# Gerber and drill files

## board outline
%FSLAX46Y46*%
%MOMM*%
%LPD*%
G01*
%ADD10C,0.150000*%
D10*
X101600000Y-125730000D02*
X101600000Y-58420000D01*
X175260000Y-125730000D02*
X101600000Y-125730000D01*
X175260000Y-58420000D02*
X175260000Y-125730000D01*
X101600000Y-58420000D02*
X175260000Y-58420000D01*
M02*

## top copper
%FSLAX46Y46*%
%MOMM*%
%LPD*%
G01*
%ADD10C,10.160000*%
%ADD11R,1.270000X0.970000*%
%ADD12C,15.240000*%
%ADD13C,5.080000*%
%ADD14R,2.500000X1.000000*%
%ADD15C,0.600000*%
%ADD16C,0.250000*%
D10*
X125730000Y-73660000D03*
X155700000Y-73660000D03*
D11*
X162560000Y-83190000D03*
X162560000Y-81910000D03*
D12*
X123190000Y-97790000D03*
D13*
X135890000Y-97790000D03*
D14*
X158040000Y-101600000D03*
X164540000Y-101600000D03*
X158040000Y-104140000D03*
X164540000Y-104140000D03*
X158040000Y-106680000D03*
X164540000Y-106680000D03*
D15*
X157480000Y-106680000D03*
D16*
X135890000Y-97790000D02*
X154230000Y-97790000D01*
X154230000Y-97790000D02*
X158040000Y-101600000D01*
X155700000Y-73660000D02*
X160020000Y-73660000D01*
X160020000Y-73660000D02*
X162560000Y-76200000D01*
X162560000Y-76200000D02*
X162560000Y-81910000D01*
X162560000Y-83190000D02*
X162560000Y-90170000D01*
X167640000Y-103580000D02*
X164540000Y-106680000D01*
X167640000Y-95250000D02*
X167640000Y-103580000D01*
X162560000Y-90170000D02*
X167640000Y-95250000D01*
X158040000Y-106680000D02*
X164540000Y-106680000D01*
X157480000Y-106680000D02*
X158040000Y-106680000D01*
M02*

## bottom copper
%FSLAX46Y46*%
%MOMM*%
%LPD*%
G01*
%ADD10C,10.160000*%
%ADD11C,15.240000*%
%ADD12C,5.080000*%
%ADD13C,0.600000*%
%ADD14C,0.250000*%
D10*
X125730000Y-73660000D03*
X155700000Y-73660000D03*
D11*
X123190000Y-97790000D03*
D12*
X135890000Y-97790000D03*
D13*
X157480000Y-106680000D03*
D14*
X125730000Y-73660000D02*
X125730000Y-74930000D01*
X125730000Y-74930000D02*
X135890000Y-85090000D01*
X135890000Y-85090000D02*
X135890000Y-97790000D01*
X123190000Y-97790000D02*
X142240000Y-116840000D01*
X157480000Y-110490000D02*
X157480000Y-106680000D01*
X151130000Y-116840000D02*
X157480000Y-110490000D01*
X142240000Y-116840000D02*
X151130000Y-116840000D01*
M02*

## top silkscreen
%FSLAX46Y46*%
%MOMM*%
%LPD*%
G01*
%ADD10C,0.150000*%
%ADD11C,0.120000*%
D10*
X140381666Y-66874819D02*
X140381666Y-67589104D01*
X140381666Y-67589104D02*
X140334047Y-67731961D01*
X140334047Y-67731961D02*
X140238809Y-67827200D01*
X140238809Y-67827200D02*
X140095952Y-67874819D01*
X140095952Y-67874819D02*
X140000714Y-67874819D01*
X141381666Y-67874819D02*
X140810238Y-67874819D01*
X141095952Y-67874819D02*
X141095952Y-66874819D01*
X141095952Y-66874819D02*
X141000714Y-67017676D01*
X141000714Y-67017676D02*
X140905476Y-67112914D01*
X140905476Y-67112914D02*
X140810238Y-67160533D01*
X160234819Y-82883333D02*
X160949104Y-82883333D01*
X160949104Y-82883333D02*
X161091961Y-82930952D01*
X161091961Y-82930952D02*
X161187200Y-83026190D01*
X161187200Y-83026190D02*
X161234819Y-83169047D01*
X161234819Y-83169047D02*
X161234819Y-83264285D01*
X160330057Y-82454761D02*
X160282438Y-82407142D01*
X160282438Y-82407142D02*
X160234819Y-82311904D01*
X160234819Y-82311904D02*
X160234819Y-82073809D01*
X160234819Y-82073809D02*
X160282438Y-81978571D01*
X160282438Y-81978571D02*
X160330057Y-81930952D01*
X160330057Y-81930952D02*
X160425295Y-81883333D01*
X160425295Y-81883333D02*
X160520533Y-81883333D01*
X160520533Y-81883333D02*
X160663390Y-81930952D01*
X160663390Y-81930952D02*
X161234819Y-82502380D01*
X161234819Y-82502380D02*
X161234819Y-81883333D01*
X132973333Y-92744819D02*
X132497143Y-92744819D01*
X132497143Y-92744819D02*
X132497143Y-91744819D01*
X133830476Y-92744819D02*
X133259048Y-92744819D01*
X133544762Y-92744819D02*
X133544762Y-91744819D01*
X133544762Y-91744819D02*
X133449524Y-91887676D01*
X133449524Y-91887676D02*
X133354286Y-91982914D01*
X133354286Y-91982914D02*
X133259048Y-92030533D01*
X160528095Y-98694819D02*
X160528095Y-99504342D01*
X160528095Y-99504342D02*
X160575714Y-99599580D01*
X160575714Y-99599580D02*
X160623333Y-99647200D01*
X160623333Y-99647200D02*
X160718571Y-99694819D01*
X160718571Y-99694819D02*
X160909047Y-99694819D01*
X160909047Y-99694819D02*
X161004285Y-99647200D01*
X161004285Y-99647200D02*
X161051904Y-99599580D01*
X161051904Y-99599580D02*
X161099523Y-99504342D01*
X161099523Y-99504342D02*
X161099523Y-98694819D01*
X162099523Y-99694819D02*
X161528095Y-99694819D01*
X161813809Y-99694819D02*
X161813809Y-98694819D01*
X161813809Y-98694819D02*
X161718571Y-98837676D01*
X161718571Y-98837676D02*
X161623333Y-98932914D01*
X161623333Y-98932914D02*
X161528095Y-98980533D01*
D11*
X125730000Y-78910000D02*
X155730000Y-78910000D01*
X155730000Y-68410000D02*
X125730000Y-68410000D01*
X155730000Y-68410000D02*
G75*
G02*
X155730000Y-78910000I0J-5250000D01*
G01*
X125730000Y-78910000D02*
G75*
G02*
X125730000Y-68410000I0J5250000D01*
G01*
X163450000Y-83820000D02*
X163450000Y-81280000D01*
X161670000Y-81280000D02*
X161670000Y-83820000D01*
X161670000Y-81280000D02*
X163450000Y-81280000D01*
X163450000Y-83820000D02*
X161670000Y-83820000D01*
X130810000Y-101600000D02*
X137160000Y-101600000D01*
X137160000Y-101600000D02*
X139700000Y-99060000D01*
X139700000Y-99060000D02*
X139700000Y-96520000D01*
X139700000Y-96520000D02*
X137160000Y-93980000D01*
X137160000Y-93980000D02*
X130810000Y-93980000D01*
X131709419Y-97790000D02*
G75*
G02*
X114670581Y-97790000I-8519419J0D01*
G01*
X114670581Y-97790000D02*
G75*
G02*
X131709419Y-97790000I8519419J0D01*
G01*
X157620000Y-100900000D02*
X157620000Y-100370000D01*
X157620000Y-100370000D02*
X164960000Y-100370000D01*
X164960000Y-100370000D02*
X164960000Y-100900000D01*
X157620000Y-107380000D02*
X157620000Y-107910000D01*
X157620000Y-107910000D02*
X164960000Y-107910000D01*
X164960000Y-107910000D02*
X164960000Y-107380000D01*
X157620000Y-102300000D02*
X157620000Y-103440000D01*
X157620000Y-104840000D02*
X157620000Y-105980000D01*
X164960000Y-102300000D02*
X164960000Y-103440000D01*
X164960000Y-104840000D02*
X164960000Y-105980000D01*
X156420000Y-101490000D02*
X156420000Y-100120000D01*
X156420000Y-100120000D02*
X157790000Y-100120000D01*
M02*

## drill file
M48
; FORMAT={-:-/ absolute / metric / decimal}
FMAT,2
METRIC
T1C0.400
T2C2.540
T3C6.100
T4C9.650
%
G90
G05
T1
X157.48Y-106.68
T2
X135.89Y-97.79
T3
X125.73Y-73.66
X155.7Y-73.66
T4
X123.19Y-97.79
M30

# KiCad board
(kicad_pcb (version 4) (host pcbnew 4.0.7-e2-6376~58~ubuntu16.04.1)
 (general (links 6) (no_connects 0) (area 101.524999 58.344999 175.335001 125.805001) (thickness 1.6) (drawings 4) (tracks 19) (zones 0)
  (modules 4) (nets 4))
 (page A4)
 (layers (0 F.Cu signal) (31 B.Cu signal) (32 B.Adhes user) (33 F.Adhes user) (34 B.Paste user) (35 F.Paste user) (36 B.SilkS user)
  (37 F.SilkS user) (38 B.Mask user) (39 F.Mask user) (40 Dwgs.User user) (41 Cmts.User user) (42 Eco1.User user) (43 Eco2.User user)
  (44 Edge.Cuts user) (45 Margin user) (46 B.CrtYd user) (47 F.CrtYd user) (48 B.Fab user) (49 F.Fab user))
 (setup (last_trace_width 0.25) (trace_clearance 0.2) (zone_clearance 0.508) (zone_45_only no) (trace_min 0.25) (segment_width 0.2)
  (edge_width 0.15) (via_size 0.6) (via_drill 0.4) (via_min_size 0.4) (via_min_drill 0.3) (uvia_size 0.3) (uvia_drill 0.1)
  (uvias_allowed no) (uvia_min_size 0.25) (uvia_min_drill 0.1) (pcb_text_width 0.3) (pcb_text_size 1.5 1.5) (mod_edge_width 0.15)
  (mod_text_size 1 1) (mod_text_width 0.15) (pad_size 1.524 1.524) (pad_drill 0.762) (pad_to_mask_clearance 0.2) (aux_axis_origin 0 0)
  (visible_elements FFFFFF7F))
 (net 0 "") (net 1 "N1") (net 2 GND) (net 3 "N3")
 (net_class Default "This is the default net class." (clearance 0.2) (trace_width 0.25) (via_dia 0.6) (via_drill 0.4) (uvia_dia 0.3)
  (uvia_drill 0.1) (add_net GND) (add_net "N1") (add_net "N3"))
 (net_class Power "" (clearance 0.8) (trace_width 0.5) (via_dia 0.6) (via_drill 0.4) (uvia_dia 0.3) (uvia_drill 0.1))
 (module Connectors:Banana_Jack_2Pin (layer F.Cu) (at 125.73 73.66)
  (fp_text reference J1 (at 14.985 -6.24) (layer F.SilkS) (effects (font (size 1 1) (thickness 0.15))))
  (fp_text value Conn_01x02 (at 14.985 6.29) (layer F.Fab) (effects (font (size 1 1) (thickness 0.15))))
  (fp_line (start 0 5.25) (end 30 5.25) (layer F.SilkS) (width 0.12))
  (fp_line (start 30 -5.25) (end 0 -5.25) (layer F.SilkS) (width 0.12))
  (fp_arc (start 30 0) (end 30 -5.25) (angle 180) (layer F.SilkS) (width 0.12))
  (fp_arc (start 0 0) (end 0 5.25) (angle 180) (layer F.SilkS) (width 0.12))
  (pad 1 thru_hole circle (at 0 0) (size 10.16 10.16) (drill 6.1) (layers *.Cu *.Mask) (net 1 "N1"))
  (pad 2 thru_hole circle (at 29.97 0) (size 10.16 10.16) (drill 6.1) (layers *.Cu *.Mask) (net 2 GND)))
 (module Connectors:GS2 (layer F.Cu) (at 162.56 82.55 180)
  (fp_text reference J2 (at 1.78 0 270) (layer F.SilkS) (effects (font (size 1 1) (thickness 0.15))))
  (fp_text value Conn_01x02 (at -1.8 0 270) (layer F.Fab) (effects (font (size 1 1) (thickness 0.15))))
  (fp_line (start -0.89 -1.27) (end -0.89 1.27) (layer F.SilkS) (width 0.12))
  (fp_line (start 0.89 1.27) (end 0.89 -1.27) (layer F.SilkS) (width 0.12))
  (fp_line (start 0.89 1.27) (end -0.89 1.27) (layer F.SilkS) (width 0.12))
  (fp_line (start -0.89 -1.27) (end 0.89 -1.27) (layer F.SilkS) (width 0.12))
  (pad 1 smd rect (at 0 -0.64 180) (size 1.27 0.97) (layers F.Cu F.Paste F.Mask) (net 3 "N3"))
  (pad 2 smd rect (at 0 0.64 180) (size 1.27 0.97) (layers F.Cu F.Paste F.Mask) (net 2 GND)))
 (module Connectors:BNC (layer F.Cu) (at 135.89 97.79)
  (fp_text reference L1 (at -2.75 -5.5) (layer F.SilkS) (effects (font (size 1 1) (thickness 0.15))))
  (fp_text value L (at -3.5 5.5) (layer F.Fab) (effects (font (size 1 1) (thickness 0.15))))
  (fp_line (start -5.08 3.81) (end 1.27 3.81) (layer F.SilkS) (width 0.12))
  (fp_line (start 1.27 3.81) (end 3.81 1.27) (layer F.SilkS) (width 0.12))
  (fp_line (start 3.81 1.27) (end 3.81 -1.27) (layer F.SilkS) (width 0.12))
  (fp_line (start 3.81 -1.27) (end 1.27 -3.81) (layer F.SilkS) (width 0.12))
  (fp_line (start 1.27 -3.81) (end -5.08 -3.81) (layer F.SilkS) (width 0.12))
  (fp_circle (center -12.7 0) (end -5.08 3.81) (layer F.SilkS) (width 0.12))
  (pad 2 thru_hole circle (at -12.7 0) (size 15.24 15.24) (drill 9.65) (layers *.Cu *.Mask) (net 3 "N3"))
  (pad 1 thru_hole circle (at 0 0) (size 5.08 5.08) (drill 2.54) (layers *.Cu *.Mask) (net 1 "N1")))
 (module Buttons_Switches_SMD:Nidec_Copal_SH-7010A (layer F.Cu) (at 161.29 104.14)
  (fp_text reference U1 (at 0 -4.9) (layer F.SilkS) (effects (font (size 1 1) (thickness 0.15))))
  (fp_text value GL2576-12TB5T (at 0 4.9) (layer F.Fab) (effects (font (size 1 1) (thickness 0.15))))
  (fp_line (start -3.67 -3.24) (end -3.67 -3.77) (layer F.SilkS) (width 0.12))
  (fp_line (start -3.67 -3.77) (end 3.67 -3.77) (layer F.SilkS) (width 0.12))
  (fp_line (start 3.67 -3.77) (end 3.67 -3.24) (layer F.SilkS) (width 0.12))
  (fp_line (start -3.67 3.24) (end -3.67 3.77) (layer F.SilkS) (width 0.12))
  (fp_line (start -3.67 3.77) (end 3.67 3.77) (layer F.SilkS) (width 0.12))
  (fp_line (start 3.67 3.77) (end 3.67 3.24) (layer F.SilkS) (width 0.12))
  (fp_line (start -3.67 -1.84) (end -3.67 -0.7) (layer F.SilkS) (width 0.12))
  (fp_line (start -3.67 0.7) (end -3.67 1.84) (layer F.SilkS) (width 0.12))
  (fp_line (start 3.67 -1.84) (end 3.67 -0.7) (layer F.SilkS) (width 0.12))
  (fp_line (start 3.67 0.7) (end 3.67 1.84) (layer F.SilkS) (width 0.12))
  (fp_line (start -4.87 -2.65) (end -4.87 -4.02) (layer F.SilkS) (width 0.12))
  (fp_line (start -4.87 -4.02) (end -3.5 -4.02) (layer F.SilkS) (width 0.12))
  (pad 1 smd rect (at -3.25 -2.54) (size 2.5 1) (layers F.Cu F.Paste F.Mask) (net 1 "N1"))
  (pad 8 smd rect (at 3.25 -2.54) (size 2.5 1) (layers F.Cu F.Paste F.Mask))
  (pad C smd rect (at -3.25 0) (size 2.5 1) (layers F.Cu F.Paste F.Mask))
  (pad C smd rect (at 3.25 0) (size 2.5 1) (layers F.Cu F.Paste F.Mask))
  (pad 4 smd rect (at -3.25 2.54) (size 2.5 1) (layers F.Cu F.Paste F.Mask) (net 3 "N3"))
  (pad 2 smd rect (at 3.25 2.54) (size 2.5 1) (layers F.Cu F.Paste F.Mask) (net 3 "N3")))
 (gr_line (start 101.6 125.73) (end 101.6 58.42) (angle 90) (layer Edge.Cuts) (width 0.15))
 (gr_line (start 175.26 125.73) (end 101.6 125.73) (angle 90) (layer Edge.Cuts) (width 0.15))
 (gr_line (start 175.26 58.42) (end 175.26 125.73) (angle 90) (layer Edge.Cuts) (width 0.15))
 (gr_line (start 101.6 58.42) (end 175.26 58.42) (angle 90) (layer Edge.Cuts) (width 0.15))
 (segment (start 135.89 97.79) (end 154.23 97.79) (width 0.25) (layer F.Cu) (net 1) (status 400000))
 (segment (start 154.23 97.79) (end 158.04 101.6) (width 0.25) (layer F.Cu) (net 1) (status 800000))
 (segment (start 125.73 73.66) (end 125.73 74.93) (width 0.25) (layer B.Cu) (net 1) (status C00000))
 (segment (start 125.73 74.93) (end 135.89 85.09) (width 0.25) (layer B.Cu) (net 1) (status 400000))
 (segment (start 135.89 85.09) (end 135.89 97.79) (width 0.25) (layer B.Cu) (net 1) (status 800000))
 (segment (start 155.7 73.66) (end 160.02 73.66) (width 0.25) (layer F.Cu) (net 2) (status C00000))
 (segment (start 160.02 73.66) (end 162.56 76.2) (width 0.25) (layer F.Cu) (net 2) (status 400000))
 (segment (start 162.56 76.2) (end 162.56 81.91) (width 0.25) (layer F.Cu) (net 2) (status 800000))
 (segment (start 162.56 83.19) (end 162.56 90.17) (width 0.25) (layer F.Cu) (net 3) (status 400000))
 (segment (start 167.64 103.58) (end 164.54 106.68) (width 0.25) (layer F.Cu) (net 3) (status 800000))
 (segment (start 167.64 95.25) (end 167.64 103.58) (width 0.25) (layer F.Cu) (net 3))
 (segment (start 162.56 90.17) (end 167.64 95.25) (width 0.25) (layer F.Cu) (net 3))
 (segment (start 158.04 106.68) (end 164.54 106.68) (width 0.25) (layer F.Cu) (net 3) (status C00000))
 (segment (start 123.19 97.79) (end 142.24 116.84) (width 0.25) (layer B.Cu) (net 3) (status 400000))
 (segment (start 157.48 106.68) (end 158.04 106.68) (width 0.25) (layer F.Cu) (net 3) (status C00000))
 (via (at 157.48 106.68) (size 0.6) (drill 0.4) (layers F.Cu B.Cu) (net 3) (status 800000))
 (segment (start 157.48 110.49) (end 157.48 106.68) (width 0.25) (layer B.Cu) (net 3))
 (segment (start 151.13 116.84) (end 157.48 110.49) (width 0.25) (layer B.Cu) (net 3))
 (segment (start 142.24 116.84) (end 151.13 116.84) (width 0.25) (layer B.Cu) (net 3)))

